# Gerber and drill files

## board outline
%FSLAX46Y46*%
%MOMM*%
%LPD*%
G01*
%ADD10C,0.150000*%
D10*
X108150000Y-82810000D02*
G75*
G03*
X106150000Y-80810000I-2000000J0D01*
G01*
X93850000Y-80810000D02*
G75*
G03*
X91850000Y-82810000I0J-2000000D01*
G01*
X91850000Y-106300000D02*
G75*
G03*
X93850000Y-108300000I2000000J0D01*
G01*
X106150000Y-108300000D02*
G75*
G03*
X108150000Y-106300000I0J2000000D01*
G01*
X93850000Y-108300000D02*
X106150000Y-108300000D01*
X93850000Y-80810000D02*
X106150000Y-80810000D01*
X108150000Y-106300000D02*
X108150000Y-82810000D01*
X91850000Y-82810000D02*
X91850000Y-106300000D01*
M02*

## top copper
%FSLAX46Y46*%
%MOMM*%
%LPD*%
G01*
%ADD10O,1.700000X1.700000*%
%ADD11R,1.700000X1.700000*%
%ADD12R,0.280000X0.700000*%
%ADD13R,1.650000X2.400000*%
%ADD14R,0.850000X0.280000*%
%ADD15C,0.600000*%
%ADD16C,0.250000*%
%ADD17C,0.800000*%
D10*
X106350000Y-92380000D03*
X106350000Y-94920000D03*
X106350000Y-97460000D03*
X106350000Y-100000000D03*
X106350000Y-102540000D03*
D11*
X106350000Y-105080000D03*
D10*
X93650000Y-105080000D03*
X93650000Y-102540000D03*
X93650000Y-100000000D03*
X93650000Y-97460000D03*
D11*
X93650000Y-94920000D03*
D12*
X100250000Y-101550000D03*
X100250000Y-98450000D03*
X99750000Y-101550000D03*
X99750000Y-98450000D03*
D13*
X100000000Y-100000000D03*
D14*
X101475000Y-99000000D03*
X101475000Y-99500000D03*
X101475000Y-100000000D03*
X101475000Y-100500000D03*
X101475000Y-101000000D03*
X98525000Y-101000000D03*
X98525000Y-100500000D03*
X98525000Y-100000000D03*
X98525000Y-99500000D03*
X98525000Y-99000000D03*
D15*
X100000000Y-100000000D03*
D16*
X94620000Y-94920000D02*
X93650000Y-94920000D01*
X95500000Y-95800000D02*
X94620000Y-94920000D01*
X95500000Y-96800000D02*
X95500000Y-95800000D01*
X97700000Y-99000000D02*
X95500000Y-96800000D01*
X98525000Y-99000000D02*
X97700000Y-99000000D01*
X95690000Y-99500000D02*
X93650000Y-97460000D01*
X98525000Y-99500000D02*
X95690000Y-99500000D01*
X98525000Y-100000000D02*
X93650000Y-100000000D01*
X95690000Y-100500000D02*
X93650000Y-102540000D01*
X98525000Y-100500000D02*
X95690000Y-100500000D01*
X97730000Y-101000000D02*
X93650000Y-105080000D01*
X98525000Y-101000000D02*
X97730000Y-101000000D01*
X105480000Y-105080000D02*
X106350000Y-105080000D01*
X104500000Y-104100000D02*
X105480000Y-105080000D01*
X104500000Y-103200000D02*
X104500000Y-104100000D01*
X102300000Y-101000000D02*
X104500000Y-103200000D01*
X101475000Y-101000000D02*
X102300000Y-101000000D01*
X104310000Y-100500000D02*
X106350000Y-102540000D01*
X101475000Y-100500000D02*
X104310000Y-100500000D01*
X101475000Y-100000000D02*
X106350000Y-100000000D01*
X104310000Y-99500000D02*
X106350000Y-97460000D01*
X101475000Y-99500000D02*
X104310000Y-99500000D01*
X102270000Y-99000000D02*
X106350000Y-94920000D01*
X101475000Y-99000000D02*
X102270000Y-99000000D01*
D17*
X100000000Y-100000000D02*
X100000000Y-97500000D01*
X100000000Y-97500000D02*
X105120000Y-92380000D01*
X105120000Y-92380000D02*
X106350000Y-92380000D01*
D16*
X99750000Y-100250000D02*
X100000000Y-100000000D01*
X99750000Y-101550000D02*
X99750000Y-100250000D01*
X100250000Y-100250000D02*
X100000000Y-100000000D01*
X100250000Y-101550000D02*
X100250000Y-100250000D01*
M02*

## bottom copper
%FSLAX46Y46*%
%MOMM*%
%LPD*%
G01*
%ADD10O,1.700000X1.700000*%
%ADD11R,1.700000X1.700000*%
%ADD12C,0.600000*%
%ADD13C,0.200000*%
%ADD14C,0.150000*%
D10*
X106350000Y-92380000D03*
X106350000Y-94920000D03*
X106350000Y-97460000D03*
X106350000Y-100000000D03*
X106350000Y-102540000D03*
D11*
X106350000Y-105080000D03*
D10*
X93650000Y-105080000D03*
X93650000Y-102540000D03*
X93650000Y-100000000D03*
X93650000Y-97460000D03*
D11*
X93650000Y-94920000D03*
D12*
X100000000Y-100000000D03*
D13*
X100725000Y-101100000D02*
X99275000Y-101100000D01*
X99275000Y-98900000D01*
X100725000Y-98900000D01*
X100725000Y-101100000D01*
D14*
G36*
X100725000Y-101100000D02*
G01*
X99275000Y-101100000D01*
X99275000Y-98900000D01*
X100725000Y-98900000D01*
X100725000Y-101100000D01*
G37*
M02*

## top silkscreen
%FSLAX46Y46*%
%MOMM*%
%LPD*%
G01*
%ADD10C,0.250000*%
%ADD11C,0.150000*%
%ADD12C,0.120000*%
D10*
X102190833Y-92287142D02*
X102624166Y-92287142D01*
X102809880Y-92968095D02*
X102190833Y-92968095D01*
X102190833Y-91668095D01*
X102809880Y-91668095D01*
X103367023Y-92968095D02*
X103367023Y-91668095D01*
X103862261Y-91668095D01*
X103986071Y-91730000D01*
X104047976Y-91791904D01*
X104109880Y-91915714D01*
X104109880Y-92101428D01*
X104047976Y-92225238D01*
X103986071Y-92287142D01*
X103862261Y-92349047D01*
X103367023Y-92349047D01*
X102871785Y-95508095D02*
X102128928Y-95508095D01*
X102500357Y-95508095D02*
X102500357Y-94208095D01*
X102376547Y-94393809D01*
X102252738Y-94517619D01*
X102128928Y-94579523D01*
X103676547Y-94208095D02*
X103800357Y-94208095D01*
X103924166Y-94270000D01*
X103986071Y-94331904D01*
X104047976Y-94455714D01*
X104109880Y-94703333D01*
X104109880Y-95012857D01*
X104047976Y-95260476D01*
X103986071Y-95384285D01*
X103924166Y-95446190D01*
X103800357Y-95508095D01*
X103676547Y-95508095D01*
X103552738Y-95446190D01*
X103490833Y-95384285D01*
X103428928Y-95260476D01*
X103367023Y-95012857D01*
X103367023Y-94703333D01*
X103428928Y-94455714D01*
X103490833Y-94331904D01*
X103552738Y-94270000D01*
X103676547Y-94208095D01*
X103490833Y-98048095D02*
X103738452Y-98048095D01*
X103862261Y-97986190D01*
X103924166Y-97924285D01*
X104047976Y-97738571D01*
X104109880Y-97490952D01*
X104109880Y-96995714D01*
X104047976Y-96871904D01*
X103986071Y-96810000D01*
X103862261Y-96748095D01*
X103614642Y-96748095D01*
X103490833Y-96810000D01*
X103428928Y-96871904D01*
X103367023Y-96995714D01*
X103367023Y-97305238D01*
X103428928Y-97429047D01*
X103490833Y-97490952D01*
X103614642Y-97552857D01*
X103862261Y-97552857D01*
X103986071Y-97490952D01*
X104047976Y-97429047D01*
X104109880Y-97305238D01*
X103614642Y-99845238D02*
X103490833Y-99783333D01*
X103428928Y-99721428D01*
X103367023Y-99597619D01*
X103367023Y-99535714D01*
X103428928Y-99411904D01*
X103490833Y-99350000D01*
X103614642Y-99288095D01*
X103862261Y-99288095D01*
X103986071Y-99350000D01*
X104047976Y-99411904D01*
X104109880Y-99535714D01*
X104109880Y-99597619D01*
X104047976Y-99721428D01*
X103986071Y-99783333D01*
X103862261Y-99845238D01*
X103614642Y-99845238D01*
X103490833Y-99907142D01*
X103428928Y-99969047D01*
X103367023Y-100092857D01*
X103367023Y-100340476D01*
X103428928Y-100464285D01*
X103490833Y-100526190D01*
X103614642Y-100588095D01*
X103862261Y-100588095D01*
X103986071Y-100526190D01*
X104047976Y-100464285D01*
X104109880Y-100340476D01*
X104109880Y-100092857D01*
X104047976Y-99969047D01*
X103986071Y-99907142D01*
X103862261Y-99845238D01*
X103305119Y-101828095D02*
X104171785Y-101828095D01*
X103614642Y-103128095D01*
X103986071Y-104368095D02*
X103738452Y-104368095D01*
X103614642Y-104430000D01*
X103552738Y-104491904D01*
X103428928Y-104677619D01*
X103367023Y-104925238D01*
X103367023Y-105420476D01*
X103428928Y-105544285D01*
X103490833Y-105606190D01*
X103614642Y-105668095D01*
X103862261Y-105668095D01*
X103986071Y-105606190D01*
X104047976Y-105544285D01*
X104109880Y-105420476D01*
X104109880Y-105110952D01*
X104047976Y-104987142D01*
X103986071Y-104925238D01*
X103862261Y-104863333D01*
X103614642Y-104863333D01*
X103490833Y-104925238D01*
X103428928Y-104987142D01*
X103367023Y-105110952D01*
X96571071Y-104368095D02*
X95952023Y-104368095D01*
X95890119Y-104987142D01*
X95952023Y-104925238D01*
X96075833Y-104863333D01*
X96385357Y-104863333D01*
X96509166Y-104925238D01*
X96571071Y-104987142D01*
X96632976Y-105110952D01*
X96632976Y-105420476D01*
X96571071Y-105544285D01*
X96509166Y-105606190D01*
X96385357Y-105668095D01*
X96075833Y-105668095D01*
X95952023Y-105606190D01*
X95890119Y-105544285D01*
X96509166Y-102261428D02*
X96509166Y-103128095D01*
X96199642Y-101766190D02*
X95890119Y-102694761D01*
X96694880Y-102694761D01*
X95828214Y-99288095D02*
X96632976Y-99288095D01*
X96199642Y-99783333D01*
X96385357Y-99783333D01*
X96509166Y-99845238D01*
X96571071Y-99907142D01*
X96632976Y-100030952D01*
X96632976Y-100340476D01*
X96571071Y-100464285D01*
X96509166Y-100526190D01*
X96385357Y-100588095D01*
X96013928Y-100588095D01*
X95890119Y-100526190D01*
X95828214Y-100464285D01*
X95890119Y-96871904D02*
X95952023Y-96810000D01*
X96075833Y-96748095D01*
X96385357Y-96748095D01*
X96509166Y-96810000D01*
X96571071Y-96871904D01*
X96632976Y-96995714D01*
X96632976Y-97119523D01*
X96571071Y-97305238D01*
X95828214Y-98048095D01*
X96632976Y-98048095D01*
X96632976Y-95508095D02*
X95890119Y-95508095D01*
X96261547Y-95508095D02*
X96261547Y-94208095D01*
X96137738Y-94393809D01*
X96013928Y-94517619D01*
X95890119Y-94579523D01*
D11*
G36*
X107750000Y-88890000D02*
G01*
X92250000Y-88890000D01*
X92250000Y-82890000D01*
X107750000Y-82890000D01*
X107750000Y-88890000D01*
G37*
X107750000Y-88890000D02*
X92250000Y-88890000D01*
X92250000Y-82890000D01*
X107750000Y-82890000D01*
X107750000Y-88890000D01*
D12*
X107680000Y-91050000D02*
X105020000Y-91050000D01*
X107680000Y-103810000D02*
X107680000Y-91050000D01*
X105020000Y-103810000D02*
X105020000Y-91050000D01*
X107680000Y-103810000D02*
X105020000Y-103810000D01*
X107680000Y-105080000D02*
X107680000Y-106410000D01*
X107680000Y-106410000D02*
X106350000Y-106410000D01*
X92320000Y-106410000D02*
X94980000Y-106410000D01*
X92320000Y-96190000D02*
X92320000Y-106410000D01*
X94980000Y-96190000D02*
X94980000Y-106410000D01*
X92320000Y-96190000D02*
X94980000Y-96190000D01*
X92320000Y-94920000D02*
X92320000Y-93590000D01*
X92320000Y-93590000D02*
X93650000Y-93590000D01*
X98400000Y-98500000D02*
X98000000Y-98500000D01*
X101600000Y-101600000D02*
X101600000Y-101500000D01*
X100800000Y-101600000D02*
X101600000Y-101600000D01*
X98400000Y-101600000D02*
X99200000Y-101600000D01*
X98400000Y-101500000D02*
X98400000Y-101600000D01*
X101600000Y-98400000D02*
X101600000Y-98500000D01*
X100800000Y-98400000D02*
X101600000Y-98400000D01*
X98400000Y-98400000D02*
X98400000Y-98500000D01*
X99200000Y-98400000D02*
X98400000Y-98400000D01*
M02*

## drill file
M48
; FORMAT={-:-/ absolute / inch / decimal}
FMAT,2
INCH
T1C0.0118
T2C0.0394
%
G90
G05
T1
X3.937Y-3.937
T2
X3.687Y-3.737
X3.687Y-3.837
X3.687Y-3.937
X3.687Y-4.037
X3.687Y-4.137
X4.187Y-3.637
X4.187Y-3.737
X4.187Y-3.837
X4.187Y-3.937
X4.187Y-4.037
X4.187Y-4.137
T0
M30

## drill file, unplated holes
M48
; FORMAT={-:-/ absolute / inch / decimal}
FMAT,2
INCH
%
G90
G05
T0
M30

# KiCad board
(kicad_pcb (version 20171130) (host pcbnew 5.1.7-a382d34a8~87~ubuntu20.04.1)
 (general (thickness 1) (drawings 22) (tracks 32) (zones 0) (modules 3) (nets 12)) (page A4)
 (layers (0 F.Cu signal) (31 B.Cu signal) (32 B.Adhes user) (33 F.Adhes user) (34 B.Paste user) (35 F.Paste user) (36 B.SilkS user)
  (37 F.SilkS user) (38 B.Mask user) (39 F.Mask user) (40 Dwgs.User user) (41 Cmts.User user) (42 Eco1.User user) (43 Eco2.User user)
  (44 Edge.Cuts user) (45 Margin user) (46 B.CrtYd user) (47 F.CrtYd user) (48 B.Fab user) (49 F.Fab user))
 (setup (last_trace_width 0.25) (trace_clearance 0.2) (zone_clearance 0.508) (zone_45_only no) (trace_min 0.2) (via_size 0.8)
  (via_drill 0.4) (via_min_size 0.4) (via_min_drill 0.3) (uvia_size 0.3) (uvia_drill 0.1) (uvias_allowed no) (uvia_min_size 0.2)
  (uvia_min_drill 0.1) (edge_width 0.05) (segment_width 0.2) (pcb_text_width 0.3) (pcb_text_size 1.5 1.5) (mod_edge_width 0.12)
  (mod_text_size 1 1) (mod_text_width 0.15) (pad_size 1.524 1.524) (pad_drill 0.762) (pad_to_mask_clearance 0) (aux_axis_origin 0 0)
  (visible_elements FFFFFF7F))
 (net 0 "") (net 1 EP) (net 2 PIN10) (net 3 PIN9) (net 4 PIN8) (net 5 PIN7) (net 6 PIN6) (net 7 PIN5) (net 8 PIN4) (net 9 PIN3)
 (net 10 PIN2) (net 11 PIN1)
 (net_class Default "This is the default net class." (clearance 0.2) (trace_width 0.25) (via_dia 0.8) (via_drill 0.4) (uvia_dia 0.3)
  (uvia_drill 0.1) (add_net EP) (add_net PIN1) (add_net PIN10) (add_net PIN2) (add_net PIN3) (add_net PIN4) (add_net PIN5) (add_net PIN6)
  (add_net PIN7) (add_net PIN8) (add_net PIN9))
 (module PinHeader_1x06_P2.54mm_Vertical (layer F.Cu) (at 106.35 105.08 180)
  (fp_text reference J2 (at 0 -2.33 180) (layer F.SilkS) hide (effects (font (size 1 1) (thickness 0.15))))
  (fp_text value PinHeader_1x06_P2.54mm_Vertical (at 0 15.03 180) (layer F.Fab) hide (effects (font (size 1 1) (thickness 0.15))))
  (fp_line (start -1.33 -1.33) (end 0 -1.33) (layer F.SilkS) (width 0.12))
  (fp_line (start -1.33 0) (end -1.33 -1.33) (layer F.SilkS) (width 0.12))
  (fp_line (start -1.33 1.27) (end 1.33 1.27) (layer F.SilkS) (width 0.12))
  (fp_line (start 1.33 1.27) (end 1.33 14.03) (layer F.SilkS) (width 0.12))
  (fp_line (start -1.33 1.27) (end -1.33 14.03) (layer F.SilkS) (width 0.12))
  (fp_line (start -1.33 14.03) (end 1.33 14.03) (layer F.SilkS) (width 0.12))
  (pad 6 thru_hole oval (at 0 12.7 180) (size 1.7 1.7) (drill 1) (layers *.Cu *.Mask) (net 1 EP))
  (pad 5 thru_hole oval (at 0 10.16 180) (size 1.7 1.7) (drill 1) (layers *.Cu *.Mask) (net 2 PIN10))
  (pad 4 thru_hole oval (at 0 7.62 180) (size 1.7 1.7) (drill 1) (layers *.Cu *.Mask) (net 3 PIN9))
  (pad 3 thru_hole oval (at 0 5.08 180) (size 1.7 1.7) (drill 1) (layers *.Cu *.Mask) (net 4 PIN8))
  (pad 2 thru_hole oval (at 0 2.54 180) (size 1.7 1.7) (drill 1) (layers *.Cu *.Mask) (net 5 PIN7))
  (pad 1 thru_hole rect (at 0 0 180) (size 1.7 1.7) (drill 1) (layers *.Cu *.Mask) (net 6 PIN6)))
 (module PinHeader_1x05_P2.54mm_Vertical (layer F.Cu) (at 93.65 94.92)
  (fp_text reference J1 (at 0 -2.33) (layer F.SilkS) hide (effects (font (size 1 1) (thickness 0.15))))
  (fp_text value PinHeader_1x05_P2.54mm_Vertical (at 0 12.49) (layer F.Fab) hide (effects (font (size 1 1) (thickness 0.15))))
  (fp_line (start -1.33 -1.33) (end 0 -1.33) (layer F.SilkS) (width 0.12))
  (fp_line (start -1.33 0) (end -1.33 -1.33) (layer F.SilkS) (width 0.12))
  (fp_line (start -1.33 1.27) (end 1.33 1.27) (layer F.SilkS) (width 0.12))
  (fp_line (start 1.33 1.27) (end 1.33 11.49) (layer F.SilkS) (width 0.12))
  (fp_line (start -1.33 1.27) (end -1.33 11.49) (layer F.SilkS) (width 0.12))
  (fp_line (start -1.33 11.49) (end 1.33 11.49) (layer F.SilkS) (width 0.12))
  (pad 5 thru_hole oval (at 0 10.16) (size 1.7 1.7) (drill 1) (layers *.Cu *.Mask) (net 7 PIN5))
  (pad 4 thru_hole oval (at 0 7.62) (size 1.7 1.7) (drill 1) (layers *.Cu *.Mask) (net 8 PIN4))
  (pad 3 thru_hole oval (at 0 5.08) (size 1.7 1.7) (drill 1) (layers *.Cu *.Mask) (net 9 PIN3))
  (pad 2 thru_hole oval (at 0 2.54) (size 1.7 1.7) (drill 1) (layers *.Cu *.Mask) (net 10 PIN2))
  (pad 1 thru_hole rect (at 0 0) (size 1.7 1.7) (drill 1) (layers *.Cu *.Mask) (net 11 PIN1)))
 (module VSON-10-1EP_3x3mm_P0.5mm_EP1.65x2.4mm (layer F.Cu) (at 100 100)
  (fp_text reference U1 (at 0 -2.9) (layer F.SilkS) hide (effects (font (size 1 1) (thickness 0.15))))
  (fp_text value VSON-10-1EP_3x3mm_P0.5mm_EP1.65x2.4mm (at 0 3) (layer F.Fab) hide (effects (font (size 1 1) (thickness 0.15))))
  (fp_line (start -0.8 -1.6) (end -1.6 -1.6) (layer F.SilkS) (width 0.12))
  (fp_line (start -1.6 -1.6) (end -1.6 -1.5) (layer F.SilkS) (width 0.12))
  (fp_line (start 0.8 -1.6) (end 1.6 -1.6) (layer F.SilkS) (width 0.12))
  (fp_line (start 1.6 -1.6) (end 1.6 -1.5) (layer F.SilkS) (width 0.12))
  (fp_line (start -1.6 1.5) (end -1.6 1.6) (layer F.SilkS) (width 0.12))
  (fp_line (start -1.6 1.6) (end -0.8 1.6) (layer F.SilkS) (width 0.12))
  (fp_line (start 0.8 1.6) (end 1.6 1.6) (layer F.SilkS) (width 0.12))
  (fp_line (start 1.6 1.6) (end 1.6 1.5) (layer F.SilkS) (width 0.12))
  (fp_line (start -1.6 -1.5) (end -2 -1.5) (layer F.SilkS) (width 0.12))
  (pad "" smd rect (at 0.4125 -0.8) (size 0.64 0.64) (layers F.Paste))
  (pad "" smd rect (at -0.4125 -0.8) (size 0.64 0.64) (layers F.Paste))
  (pad "" smd rect (at 0.4125 0) (size 0.64 0.64) (layers F.Paste))
  (pad "" smd rect (at -0.4125 0) (size 0.64 0.64) (layers F.Paste))
  (pad "" smd rect (at -0.4125 0.8) (size 0.64 0.64) (layers F.Paste))
  (pad 11 smd rect (at 0.25 1.55) (size 0.28 0.7) (layers F.Cu F.Paste F.Mask) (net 1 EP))
  (pad 11 smd rect (at 0.25 -1.55) (size 0.28 0.7) (layers F.Cu F.Paste F.Mask) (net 1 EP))
  (pad 11 smd rect (at -0.25 1.55) (size 0.28 0.7) (layers F.Cu F.Paste F.Mask) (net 1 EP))
  (pad 11 smd rect (at -0.25 -1.55) (size 0.28 0.7) (layers F.Cu F.Paste F.Mask) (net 1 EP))
  (pad "" smd rect (at 0.4125 0.8) (size 0.64 0.64) (layers F.Paste))
  (pad 11 smd rect (at 0 0) (size 1.65 2.4) (layers F.Cu F.Mask) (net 1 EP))
  (pad 10 smd rect (at 1.475 -1) (size 0.85 0.28) (layers F.Cu F.Paste F.Mask) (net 2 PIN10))
  (pad 9 smd rect (at 1.475 -0.5) (size 0.85 0.28) (layers F.Cu F.Paste F.Mask) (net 3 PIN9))
  (pad 8 smd rect (at 1.475 0) (size 0.85 0.28) (layers F.Cu F.Paste F.Mask) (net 4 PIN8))
  (pad 7 smd rect (at 1.475 0.5) (size 0.85 0.28) (layers F.Cu F.Paste F.Mask) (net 5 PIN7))
  (pad 6 smd rect (at 1.475 1) (size 0.85 0.28) (layers F.Cu F.Paste F.Mask) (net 6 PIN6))
  (pad 5 smd rect (at -1.475 1) (size 0.85 0.28) (layers F.Cu F.Paste F.Mask) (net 7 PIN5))
  (pad 4 smd rect (at -1.475 0.5) (size 0.85 0.28) (layers F.Cu F.Paste F.Mask) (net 8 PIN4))
  (pad 3 smd rect (at -1.475 0) (size 0.85 0.28) (layers F.Cu F.Paste F.Mask) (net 9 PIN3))
  (pad 2 smd rect (at -1.475 -0.5) (size 0.85 0.28) (layers F.Cu F.Paste F.Mask) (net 10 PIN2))
  (pad 1 smd rect (at -1.475 -1) (size 0.85 0.28) (layers F.Cu F.Paste F.Mask) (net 11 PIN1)))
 (gr_arc (start 106.15 82.81) (end 106.15 80.81) (angle 90) (layer Edge.Cuts) (width 0.15))
 (gr_arc (start 93.85 82.81) (end 91.85 82.81) (angle 90) (layer Edge.Cuts) (width 0.15))
 (gr_arc (start 93.85 106.3) (end 93.85 108.3) (angle 90) (layer Edge.Cuts) (width 0.15))
 (gr_arc (start 106.15 106.3) (end 108.15 106.3) (angle 90) (layer Edge.Cuts) (width 0.15))
 (gr_line (start 93.85 108.3) (end 106.15 108.3) (layer Edge.Cuts) (width 0.15))
 (gr_line (start 93.85 80.81) (end 106.15 80.81) (layer Edge.Cuts) (width 0.15))
 (gr_line (start 108.15 106.3) (end 108.15 82.81) (layer Edge.Cuts) (width 0.15))
 (gr_line (start 91.85 82.81) (end 91.85 106.3) (layer Edge.Cuts) (width 0.15))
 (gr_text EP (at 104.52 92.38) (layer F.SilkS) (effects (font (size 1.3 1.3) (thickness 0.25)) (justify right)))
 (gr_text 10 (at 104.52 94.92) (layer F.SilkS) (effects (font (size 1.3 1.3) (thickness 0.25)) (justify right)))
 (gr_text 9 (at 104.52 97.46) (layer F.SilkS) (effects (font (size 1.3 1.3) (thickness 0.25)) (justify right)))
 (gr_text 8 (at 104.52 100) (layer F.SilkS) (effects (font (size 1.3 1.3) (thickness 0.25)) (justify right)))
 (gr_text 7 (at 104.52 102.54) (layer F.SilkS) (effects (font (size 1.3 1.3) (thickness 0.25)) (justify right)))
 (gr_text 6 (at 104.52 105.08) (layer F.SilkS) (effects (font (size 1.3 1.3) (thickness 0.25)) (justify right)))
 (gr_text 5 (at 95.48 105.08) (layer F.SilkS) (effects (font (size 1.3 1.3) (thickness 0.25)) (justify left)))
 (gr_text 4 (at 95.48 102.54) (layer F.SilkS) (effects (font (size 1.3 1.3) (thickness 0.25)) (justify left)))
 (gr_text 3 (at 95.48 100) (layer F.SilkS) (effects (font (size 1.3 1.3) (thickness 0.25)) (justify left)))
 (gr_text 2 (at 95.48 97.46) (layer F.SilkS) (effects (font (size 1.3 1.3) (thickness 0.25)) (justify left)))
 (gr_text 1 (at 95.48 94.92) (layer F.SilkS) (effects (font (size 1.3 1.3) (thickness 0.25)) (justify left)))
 (gr_poly (pts (xy 92.25 82.89) (xy 92.25 88.89) (xy 107.75 88.89) (xy 107.75 82.89)) (layer F.SilkS) (width 0.15))
 (segment (start 94.62 94.92) (end 93.65 94.92) (width 0.25) (layer F.Cu) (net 11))
 (segment (start 95.5 95.8) (end 94.62 94.92) (width 0.25) (layer F.Cu) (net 11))
 (segment (start 95.5 96.8) (end 95.5 95.8) (width 0.25) (layer F.Cu) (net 11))
 (segment (start 97.7 99) (end 95.5 96.8) (width 0.25) (layer F.Cu) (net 11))
 (segment (start 98.525 99) (end 97.7 99) (width 0.25) (layer F.Cu) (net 11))
 (segment (start 95.69 99.5) (end 93.65 97.46) (width 0.25) (layer F.Cu) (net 10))
 (segment (start 98.525 99.5) (end 95.69 99.5) (width 0.25) (layer F.Cu) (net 10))
 (segment (start 98.525 100) (end 93.65 100) (width 0.25) (layer F.Cu) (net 9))
 (segment (start 95.69 100.5) (end 93.65 102.54) (width 0.25) (layer F.Cu) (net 8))
 (segment (start 98.525 100.5) (end 95.69 100.5) (width 0.25) (layer F.Cu) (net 8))
 (segment (start 97.73 101) (end 93.65 105.08) (width 0.25) (layer F.Cu) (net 7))
 (segment (start 98.525 101) (end 97.73 101) (width 0.25) (layer F.Cu) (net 7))
 (segment (start 105.48 105.08) (end 106.35 105.08) (width 0.25) (layer F.Cu) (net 6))
 (segment (start 104.5 104.1) (end 105.48 105.08) (width 0.25) (layer F.Cu) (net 6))
 (segment (start 104.5 103.2) (end 104.5 104.1) (width 0.25) (layer F.Cu) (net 6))
 (segment (start 102.3 101) (end 104.5 103.2) (width 0.25) (layer F.Cu) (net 6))
 (segment (start 101.475 101) (end 102.3 101) (width 0.25) (layer F.Cu) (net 6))
 (segment (start 104.31 100.5) (end 106.35 102.54) (width 0.25) (layer F.Cu) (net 5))
 (segment (start 101.475 100.5) (end 104.31 100.5) (width 0.25) (layer F.Cu) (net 5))
 (segment (start 101.475 100) (end 106.35 100) (width 0.25) (layer F.Cu) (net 4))
 (segment (start 104.31 99.5) (end 106.35 97.46) (width 0.25) (layer F.Cu) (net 3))
 (segment (start 101.475 99.5) (end 104.31 99.5) (width 0.25) (layer F.Cu) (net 3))
 (segment (start 102.27 99) (end 106.35 94.92) (width 0.25) (layer F.Cu) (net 2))
 (segment (start 101.475 99) (end 102.27 99) (width 0.25) (layer F.Cu) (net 2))
 (via (at 100 100) (size 0.6) (drill 0.3) (layers F.Cu B.Cu) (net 1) (status 1000000))
 (segment (start 100 100) (end 100 97.5) (width 0.8) (layer F.Cu) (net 1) (status 1000000))
 (segment (start 100 97.5) (end 105.12 92.38) (width 0.8) (layer F.Cu) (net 1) (status 1000000))
 (segment (start 105.12 92.38) (end 106.35 92.38) (width 0.8) (layer F.Cu) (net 1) (status 1000000))
 (segment (start 99.75 100.25) (end 100 100) (width 0.25) (layer F.Cu) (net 1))
 (segment (start 99.75 101.55) (end 99.75 100.25) (width 0.25) (layer F.Cu) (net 1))
 (segment (start 100.25 100.25) (end 100 100) (width 0.25) (layer F.Cu) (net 1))
 (segment (start 100.25 101.55) (end 100.25 100.25) (width 0.25) (layer F.Cu) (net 1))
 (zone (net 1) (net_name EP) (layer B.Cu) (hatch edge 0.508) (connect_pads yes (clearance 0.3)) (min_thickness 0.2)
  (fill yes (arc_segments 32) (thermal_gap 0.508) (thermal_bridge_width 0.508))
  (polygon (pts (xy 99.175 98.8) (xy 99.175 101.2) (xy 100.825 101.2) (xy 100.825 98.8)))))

